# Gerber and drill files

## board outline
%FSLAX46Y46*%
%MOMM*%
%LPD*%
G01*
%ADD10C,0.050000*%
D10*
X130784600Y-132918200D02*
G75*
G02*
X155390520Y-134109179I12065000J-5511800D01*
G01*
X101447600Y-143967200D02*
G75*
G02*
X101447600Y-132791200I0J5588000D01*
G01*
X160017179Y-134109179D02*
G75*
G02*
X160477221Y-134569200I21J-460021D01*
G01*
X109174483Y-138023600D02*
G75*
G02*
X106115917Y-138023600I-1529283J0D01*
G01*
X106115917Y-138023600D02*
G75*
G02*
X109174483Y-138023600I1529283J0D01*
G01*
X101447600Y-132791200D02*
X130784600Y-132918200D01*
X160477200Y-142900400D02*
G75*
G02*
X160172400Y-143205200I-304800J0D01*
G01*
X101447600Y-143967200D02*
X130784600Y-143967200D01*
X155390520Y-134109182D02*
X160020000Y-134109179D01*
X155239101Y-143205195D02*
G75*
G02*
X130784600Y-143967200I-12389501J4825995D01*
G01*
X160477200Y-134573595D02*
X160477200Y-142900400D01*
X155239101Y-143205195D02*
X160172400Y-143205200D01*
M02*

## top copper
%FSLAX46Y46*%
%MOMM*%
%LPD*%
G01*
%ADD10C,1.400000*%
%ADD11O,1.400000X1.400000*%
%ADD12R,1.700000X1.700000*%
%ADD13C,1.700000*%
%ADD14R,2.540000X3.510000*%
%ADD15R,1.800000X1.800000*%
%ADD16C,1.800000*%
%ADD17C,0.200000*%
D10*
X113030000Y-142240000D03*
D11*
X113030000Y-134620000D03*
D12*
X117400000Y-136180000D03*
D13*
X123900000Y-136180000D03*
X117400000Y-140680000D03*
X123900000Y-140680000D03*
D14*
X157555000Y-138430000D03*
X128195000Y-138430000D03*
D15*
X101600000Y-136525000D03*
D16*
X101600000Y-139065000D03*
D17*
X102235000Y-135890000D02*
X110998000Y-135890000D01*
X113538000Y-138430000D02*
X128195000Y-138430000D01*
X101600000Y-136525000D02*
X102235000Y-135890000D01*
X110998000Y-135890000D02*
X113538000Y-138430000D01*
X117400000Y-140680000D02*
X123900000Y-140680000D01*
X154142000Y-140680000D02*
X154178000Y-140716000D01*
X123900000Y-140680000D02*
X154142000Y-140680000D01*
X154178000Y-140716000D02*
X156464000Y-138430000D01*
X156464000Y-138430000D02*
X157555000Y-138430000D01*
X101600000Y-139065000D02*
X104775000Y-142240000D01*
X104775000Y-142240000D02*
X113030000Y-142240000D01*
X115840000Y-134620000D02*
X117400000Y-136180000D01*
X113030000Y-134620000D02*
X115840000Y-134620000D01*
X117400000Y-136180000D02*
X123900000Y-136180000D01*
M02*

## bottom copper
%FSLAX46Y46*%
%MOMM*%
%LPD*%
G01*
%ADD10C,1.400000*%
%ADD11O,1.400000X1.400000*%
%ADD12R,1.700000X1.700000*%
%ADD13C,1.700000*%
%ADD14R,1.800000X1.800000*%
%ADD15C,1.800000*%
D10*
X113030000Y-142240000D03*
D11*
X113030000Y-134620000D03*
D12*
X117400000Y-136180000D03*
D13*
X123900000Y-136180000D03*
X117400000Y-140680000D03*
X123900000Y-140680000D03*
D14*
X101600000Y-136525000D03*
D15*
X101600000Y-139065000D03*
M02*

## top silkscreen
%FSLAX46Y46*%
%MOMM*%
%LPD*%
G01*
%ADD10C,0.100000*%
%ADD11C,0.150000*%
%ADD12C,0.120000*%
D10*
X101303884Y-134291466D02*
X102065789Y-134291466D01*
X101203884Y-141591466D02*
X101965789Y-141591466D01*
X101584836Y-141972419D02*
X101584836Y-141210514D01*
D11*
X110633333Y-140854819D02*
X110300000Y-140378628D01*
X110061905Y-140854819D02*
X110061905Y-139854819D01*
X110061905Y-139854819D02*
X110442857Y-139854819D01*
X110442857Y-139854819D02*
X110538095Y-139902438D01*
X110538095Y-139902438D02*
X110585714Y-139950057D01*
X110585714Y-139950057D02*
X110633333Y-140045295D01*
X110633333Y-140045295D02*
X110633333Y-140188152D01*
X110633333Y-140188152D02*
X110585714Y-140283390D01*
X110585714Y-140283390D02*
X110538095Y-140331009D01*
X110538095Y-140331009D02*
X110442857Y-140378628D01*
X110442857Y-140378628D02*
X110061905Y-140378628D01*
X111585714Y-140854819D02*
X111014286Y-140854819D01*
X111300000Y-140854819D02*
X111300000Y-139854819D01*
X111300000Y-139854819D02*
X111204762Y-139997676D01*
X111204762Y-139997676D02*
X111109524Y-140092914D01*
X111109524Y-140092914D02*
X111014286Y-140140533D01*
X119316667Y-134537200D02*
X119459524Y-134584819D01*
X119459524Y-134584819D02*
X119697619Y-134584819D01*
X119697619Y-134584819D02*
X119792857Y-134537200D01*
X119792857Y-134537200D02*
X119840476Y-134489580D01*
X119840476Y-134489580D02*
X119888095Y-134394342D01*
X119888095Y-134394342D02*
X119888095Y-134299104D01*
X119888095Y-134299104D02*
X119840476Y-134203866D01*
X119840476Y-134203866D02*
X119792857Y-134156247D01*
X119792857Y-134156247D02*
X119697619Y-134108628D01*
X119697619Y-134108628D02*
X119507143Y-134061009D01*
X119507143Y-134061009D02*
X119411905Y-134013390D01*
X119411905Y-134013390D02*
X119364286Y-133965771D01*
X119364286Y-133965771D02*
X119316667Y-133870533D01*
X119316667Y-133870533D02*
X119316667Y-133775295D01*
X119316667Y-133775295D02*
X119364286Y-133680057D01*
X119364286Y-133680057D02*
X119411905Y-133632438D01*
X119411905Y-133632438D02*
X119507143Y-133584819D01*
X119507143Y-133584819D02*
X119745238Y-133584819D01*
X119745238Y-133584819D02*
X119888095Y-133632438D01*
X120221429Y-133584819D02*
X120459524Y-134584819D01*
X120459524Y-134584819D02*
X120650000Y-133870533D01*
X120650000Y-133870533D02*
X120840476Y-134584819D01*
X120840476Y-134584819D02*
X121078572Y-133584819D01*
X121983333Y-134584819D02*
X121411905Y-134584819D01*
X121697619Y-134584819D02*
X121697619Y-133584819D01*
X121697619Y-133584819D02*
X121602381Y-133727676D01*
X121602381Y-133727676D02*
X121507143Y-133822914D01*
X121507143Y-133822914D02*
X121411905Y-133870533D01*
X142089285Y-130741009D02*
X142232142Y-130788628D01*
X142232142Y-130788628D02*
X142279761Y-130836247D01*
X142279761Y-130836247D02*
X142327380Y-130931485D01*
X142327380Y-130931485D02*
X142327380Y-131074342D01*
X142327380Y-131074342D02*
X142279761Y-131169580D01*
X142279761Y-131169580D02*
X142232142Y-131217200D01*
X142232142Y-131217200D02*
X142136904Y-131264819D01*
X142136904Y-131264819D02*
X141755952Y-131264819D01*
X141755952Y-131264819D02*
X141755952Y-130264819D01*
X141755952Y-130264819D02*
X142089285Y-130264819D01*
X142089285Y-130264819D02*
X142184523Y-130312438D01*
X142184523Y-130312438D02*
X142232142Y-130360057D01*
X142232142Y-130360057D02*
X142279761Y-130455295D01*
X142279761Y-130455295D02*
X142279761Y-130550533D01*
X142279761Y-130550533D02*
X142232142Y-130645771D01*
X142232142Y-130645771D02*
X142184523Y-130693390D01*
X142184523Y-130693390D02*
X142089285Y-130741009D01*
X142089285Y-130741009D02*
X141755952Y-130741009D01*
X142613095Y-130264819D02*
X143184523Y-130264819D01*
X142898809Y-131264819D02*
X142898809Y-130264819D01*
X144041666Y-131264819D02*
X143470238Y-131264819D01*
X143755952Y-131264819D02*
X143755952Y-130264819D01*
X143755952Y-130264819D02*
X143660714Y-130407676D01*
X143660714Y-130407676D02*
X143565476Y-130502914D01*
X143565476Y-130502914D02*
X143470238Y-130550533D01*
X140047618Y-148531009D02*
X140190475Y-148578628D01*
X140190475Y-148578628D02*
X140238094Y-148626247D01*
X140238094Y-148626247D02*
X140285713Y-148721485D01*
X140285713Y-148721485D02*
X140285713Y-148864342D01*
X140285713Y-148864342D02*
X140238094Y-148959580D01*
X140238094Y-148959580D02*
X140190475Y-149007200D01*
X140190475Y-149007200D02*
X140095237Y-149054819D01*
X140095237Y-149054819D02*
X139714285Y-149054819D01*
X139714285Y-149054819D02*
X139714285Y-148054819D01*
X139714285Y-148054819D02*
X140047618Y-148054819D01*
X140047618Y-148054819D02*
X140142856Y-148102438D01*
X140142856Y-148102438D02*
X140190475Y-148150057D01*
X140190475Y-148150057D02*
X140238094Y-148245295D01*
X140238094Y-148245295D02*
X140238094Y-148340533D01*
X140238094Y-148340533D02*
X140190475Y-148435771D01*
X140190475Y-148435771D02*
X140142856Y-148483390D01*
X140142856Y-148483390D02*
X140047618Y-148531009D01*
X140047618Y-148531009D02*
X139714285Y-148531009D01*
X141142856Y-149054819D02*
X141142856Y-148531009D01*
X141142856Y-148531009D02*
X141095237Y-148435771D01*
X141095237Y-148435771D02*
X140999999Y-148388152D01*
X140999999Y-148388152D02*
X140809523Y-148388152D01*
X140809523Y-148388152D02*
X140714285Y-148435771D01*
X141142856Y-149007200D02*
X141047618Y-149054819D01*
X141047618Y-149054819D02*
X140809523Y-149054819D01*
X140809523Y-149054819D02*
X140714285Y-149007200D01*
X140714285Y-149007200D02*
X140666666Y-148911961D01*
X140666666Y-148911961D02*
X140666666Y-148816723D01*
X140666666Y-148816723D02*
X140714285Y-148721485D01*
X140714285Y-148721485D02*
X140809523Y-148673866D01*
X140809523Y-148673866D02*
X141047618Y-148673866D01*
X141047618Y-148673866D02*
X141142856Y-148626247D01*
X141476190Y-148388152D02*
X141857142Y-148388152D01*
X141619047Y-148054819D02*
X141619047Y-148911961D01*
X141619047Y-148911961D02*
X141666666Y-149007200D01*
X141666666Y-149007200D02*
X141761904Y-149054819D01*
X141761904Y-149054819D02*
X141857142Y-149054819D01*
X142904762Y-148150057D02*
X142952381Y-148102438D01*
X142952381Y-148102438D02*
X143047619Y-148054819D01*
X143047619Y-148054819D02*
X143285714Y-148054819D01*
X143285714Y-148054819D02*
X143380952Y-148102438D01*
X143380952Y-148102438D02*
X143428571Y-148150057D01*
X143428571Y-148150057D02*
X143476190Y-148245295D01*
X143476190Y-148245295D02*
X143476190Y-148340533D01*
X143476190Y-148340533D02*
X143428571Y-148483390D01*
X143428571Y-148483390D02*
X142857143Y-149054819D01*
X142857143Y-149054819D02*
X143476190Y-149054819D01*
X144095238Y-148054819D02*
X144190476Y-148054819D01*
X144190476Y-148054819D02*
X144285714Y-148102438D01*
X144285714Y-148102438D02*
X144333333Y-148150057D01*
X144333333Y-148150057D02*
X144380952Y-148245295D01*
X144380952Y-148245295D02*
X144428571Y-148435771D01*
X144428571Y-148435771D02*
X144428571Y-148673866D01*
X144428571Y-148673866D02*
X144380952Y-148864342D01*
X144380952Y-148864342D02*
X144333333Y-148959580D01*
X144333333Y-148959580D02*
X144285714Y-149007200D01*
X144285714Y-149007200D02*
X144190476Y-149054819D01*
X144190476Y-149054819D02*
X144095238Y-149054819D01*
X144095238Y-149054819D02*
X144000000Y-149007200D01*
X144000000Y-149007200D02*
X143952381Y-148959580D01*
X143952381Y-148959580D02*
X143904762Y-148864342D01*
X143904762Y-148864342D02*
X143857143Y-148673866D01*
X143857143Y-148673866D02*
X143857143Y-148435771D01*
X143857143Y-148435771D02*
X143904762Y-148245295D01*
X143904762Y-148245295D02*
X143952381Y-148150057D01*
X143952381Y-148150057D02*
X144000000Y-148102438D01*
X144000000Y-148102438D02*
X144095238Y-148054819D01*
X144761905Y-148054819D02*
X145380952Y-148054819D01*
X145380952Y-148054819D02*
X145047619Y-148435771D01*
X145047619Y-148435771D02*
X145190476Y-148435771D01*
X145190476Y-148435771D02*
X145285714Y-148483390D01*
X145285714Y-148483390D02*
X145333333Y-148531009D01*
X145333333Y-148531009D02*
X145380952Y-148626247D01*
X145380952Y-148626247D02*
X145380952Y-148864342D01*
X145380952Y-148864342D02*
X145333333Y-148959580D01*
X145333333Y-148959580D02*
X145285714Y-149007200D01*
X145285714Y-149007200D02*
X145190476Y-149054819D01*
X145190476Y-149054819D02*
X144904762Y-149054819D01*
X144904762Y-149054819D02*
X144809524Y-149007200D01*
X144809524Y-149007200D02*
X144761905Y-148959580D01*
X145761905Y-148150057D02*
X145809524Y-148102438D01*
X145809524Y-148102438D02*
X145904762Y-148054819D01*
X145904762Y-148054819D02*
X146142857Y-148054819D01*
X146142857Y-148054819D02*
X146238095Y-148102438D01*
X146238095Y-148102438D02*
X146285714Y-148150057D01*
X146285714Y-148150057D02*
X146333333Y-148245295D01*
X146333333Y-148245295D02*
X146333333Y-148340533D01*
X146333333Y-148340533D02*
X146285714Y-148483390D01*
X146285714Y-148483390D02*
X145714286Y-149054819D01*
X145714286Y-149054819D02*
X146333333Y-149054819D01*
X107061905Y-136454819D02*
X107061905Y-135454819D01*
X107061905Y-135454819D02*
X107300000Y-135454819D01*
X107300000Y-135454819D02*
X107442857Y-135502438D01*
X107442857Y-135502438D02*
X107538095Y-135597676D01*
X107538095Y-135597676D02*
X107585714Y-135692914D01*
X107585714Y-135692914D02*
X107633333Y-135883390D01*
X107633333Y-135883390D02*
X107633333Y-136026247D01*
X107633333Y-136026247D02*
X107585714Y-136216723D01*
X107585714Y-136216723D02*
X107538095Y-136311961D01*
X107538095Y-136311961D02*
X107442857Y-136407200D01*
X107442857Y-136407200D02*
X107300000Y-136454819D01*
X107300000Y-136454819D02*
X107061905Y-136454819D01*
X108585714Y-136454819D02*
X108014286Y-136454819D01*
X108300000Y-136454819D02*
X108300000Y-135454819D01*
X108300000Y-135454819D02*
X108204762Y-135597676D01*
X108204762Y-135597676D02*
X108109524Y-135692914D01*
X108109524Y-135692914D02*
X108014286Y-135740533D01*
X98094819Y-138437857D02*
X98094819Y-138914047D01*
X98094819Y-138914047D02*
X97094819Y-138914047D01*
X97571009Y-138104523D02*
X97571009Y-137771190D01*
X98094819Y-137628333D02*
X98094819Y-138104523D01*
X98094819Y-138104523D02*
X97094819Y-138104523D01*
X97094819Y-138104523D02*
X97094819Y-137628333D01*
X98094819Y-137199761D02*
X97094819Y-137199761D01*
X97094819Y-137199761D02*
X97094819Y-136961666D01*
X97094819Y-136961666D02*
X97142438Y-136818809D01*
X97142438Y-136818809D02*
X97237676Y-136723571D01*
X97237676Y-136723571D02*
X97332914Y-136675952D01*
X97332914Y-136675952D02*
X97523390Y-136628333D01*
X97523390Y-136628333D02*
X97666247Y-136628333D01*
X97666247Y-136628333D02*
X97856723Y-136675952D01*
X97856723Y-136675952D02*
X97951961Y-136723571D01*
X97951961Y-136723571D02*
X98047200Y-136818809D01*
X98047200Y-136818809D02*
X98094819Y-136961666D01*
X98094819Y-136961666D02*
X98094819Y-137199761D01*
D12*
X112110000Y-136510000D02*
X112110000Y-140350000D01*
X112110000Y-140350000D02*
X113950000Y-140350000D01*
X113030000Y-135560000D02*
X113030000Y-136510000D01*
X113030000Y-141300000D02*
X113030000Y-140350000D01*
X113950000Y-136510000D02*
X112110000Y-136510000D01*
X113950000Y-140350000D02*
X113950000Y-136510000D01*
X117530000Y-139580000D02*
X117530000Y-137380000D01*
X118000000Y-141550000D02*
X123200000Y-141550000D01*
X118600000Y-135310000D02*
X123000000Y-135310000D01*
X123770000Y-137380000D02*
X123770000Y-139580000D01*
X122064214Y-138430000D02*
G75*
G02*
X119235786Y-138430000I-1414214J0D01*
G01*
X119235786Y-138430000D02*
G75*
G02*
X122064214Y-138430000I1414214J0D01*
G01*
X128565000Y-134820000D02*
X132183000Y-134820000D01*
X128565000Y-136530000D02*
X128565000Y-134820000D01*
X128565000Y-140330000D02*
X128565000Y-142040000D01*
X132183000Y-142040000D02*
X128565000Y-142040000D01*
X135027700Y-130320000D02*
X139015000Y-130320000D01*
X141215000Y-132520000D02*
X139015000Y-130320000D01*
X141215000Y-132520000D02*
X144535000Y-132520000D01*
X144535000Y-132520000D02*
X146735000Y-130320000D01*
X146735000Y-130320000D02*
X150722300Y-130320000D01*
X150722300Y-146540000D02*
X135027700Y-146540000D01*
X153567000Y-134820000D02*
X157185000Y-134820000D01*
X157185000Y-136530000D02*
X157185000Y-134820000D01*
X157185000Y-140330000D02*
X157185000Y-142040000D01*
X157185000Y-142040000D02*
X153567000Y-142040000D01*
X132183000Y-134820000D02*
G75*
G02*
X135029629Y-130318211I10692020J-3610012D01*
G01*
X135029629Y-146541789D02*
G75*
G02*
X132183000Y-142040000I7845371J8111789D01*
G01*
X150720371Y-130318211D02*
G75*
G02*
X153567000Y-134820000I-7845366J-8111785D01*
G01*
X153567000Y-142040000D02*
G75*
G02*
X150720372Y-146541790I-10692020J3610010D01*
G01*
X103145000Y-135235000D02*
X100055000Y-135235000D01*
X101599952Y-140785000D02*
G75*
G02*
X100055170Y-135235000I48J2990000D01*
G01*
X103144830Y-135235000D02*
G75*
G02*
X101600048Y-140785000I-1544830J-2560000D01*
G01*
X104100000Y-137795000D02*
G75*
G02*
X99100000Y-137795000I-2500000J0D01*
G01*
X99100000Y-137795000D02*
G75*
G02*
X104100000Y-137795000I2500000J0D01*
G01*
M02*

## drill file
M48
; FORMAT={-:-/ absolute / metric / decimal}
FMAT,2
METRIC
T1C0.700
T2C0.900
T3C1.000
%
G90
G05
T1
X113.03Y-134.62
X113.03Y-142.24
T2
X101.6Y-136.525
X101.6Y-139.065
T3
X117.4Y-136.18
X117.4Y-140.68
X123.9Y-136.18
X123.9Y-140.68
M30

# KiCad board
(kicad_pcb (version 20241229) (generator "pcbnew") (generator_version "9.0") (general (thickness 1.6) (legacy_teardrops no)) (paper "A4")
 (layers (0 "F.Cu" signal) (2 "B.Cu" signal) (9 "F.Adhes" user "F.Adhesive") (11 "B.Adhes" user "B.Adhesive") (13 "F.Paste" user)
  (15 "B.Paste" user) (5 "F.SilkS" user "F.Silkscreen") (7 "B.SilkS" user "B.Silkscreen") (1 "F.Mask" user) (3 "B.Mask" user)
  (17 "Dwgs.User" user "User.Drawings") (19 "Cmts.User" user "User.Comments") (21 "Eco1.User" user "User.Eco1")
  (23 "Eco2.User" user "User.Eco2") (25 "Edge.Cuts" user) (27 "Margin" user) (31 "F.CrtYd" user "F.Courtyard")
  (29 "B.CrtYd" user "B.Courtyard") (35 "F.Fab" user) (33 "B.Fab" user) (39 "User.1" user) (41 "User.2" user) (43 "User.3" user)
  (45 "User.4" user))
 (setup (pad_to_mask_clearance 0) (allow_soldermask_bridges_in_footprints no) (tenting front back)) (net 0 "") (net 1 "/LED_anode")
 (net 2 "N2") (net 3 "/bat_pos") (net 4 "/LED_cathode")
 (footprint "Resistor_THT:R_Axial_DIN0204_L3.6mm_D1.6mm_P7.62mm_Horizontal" (layer "F.Cu") (at 113.03 142.24 90)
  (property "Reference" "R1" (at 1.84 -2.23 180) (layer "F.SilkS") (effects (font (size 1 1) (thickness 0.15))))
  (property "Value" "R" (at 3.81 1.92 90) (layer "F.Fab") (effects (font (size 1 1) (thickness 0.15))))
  (fp_line (start 5.73 -0.92) (end 1.89 -0.92) (stroke (width 0.12) (type solid)) (layer "F.SilkS"))
  (fp_line (start 1.89 -0.92) (end 1.89 0.92) (stroke (width 0.12) (type solid)) (layer "F.SilkS"))
  (fp_line (start 6.68 0) (end 5.73 0) (stroke (width 0.12) (type solid)) (layer "F.SilkS"))
  (fp_line (start 0.94 0) (end 1.89 0) (stroke (width 0.12) (type solid)) (layer "F.SilkS"))
  (fp_line (start 5.73 0.92) (end 5.73 -0.92) (stroke (width 0.12) (type solid)) (layer "F.SilkS"))
  (fp_line (start 1.89 0.92) (end 5.73 0.92) (stroke (width 0.12) (type solid)) (layer "F.SilkS"))
  (pad "1" thru_hole circle (at 0 0 90) (size 1.4 1.4) (drill 0.7) (layers "*.Cu" "*.Mask") (remove_unused_layers no) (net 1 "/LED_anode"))
  (pad "2" thru_hole oval (at 7.62 0 90) (size 1.4 1.4) (drill 0.7) (layers "*.Cu" "*.Mask") (remove_unused_layers no) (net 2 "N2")))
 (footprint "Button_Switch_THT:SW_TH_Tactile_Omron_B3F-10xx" (layer "F.Cu") (at 117.4 136.18)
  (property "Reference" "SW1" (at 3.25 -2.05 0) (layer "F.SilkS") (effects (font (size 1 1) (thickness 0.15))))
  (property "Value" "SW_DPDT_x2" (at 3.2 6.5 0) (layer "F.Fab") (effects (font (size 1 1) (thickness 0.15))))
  (fp_line (start 0.13 3.4) (end 0.13 1.2) (stroke (width 0.12) (type solid)) (layer "F.SilkS"))
  (fp_line (start 0.6 5.37) (end 5.8 5.37) (stroke (width 0.12) (type solid)) (layer "F.SilkS"))
  (fp_line (start 1.2 -0.87) (end 5.6 -0.87) (stroke (width 0.12) (type solid)) (layer "F.SilkS"))
  (fp_line (start 6.37 1.2) (end 6.37 3.4) (stroke (width 0.12) (type solid)) (layer "F.SilkS"))
  (fp_circle (center 3.25 2.25) (end 4.25 3.25) (stroke (width 0.12) (type solid)) (fill no) (layer "F.SilkS"))
  (pad "1" thru_hole rect (at 0 0) (size 1.7 1.7) (drill 1) (layers "*.Cu" "*.Mask") (remove_unused_layers no) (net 2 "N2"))
  (pad "1" thru_hole circle (at 6.5 0) (size 1.7 1.7) (drill 1) (layers "*.Cu" "*.Mask") (remove_unused_layers no) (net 2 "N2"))
  (pad "2" thru_hole circle (at 0 4.5) (size 1.7 1.7) (drill 1) (layers "*.Cu" "*.Mask") (remove_unused_layers no) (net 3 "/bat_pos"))
  (pad "2" thru_hole circle (at 6.5 4.5) (size 1.7 1.7) (drill 1) (layers "*.Cu" "*.Mask") (remove_unused_layers no) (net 3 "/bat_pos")))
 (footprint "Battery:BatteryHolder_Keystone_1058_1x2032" (layer "F.Cu") (at 142.875 138.43 180)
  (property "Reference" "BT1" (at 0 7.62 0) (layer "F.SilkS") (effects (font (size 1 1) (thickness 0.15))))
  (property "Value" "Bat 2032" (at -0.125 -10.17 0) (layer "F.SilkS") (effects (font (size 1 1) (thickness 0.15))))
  (fp_line (start 14.31 3.61) (end 10.692 3.61) (stroke (width 0.12) (type solid)) (layer "F.SilkS"))
  (fp_line (start 14.31 1.9) (end 14.31 3.61) (stroke (width 0.12) (type solid)) (layer "F.SilkS"))
  (fp_line (start 14.31 -1.9) (end 14.31 -3.61) (stroke (width 0.12) (type solid)) (layer "F.SilkS"))
  (fp_line (start 10.692 -3.61) (end 14.31 -3.61) (stroke (width 0.12) (type solid)) (layer "F.SilkS"))
  (fp_line (start 7.8473 8.11) (end 3.86 8.11) (stroke (width 0.12) (type solid)) (layer "F.SilkS"))
  (fp_line (start 1.66 5.91) (end 3.86 8.11) (stroke (width 0.12) (type solid)) (layer "F.SilkS"))
  (fp_line (start 1.66 5.91) (end -1.66 5.91) (stroke (width 0.12) (type solid)) (layer "F.SilkS"))
  (fp_line (start -1.66 5.91) (end -3.86 8.11) (stroke (width 0.12) (type solid)) (layer "F.SilkS"))
  (fp_line (start -3.86 8.11) (end -7.8473 8.11) (stroke (width 0.12) (type solid)) (layer "F.SilkS"))
  (fp_line (start -7.8473 -8.11) (end 7.8473 -8.11) (stroke (width 0.12) (type solid)) (layer "F.SilkS"))
  (fp_line (start -10.692 3.61) (end -14.31 3.61) (stroke (width 0.12) (type solid)) (layer "F.SilkS"))
  (fp_line (start -14.31 1.9) (end -14.31 3.61) (stroke (width 0.12) (type solid)) (layer "F.SilkS"))
  (fp_line (start -14.31 -1.9) (end -14.31 -3.61) (stroke (width 0.12) (type solid)) (layer "F.SilkS"))
  (fp_line (start -14.31 -3.61) (end -10.692 -3.61) (stroke (width 0.12) (type solid)) (layer "F.SilkS"))
  (fp_arc (start 10.692 3.61) (mid 9.538084 6.031244) (end 7.845371 8.111789) (stroke (width 0.12) (type solid)) (layer "F.SilkS"))
  (fp_arc (start 7.845371 -8.111789) (mid 9.538085 -6.031244) (end 10.692 -3.61) (stroke (width 0.12) (type solid)) (layer "F.SilkS"))
  (fp_arc (start -7.845371 8.111789) (mid -9.538085 6.031244) (end -10.692 3.61) (stroke (width 0.12) (type solid)) (layer "F.SilkS"))
  (fp_arc (start -10.692 -3.61) (mid -9.538084 -6.031244) (end -7.845371 -8.111789) (stroke (width 0.12) (type solid)) (layer "F.SilkS"))
  (pad "1" smd rect (at -14.68 0 180) (size 2.54 3.51) (layers "F.Cu" "F.Mask" "F.Paste") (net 3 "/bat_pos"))
  (pad "2" smd rect (at 14.68 0 180) (size 2.54 3.51) (layers "F.Cu" "F.Mask" "F.Paste") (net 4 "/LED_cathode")))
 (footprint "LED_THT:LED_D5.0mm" (layer "F.Cu") (at 101.6 136.525 -90)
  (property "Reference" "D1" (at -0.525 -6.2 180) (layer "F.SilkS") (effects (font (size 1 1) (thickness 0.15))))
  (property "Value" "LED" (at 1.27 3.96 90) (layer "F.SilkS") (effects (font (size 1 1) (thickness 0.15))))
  (fp_line (start -1.29 -1.545) (end -1.29 1.545) (stroke (width 0.12) (type solid)) (layer "F.SilkS"))
  (fp_arc (start 4.26 0.000048) (mid 2.071756 2.880501) (end -1.29 1.54483) (stroke (width 0.12) (type solid)) (layer "F.SilkS"))
  (fp_arc (start -1.29 -1.54483) (mid 2.071756 -2.880501) (end 4.26 -0.000048) (stroke (width 0.12) (type solid)) (layer "F.SilkS"))
  (fp_circle (center 1.27 0) (end 3.77 0) (stroke (width 0.12) (type solid)) (fill no) (layer "F.SilkS"))
  (pad "1" thru_hole rect (at 0 0 270) (size 1.8 1.8) (drill 0.9) (layers "*.Cu" "*.Mask") (remove_unused_layers no) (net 4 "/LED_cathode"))
  (pad "2" thru_hole circle (at 2.54 0 270) (size 1.8 1.8) (drill 0.9) (layers "*.Cu" "*.Mask") (remove_unused_layers no)
   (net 1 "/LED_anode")))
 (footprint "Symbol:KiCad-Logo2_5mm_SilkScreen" (layer "B.Cu") (at 143.51 136.525 180)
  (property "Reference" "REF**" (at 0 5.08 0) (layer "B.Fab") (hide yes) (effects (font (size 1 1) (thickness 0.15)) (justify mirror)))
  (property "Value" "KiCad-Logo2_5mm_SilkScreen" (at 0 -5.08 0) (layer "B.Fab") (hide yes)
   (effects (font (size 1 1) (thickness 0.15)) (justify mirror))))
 (gr_arc (start 130.7846 132.9182) (mid 143.490874 125.181116) (end 155.39052 134.109179) (stroke (width 0.05) (type default)) (locked yes)
  (layer "Edge.Cuts"))
 (gr_arc (start 101.4476 143.9672) (mid 95.8596 138.3792) (end 101.4476 132.7912) (stroke (width 0.05) (type default)) (locked yes)
  (layer "Edge.Cuts"))
 (gr_arc (start 160.017179 134.109179) (mid 160.342463 134.243916) (end 160.4772 134.5692) (stroke (width 0.05) (type default)) (locked yes)
  (layer "Edge.Cuts"))
 (gr_circle (center 107.6452 138.0236) (end 108.7882 139.0396) (stroke (width 0.05) (type default)) (fill no) (layer "Edge.Cuts"))
 (gr_line (start 101.4476 132.7912) (end 130.7846 132.9182) (stroke (width 0.05) (type default)) (locked yes) (layer "Edge.Cuts"))
 (gr_arc (start 160.4772 142.9004) (mid 160.387926 143.115926) (end 160.1724 143.2052) (stroke (width 0.05) (type default)) (locked yes)
  (layer "Edge.Cuts"))
 (gr_line (start 101.4476 143.9672) (end 130.7846 143.9672) (stroke (width 0.05) (type default)) (locked yes) (layer "Edge.Cuts"))
 (gr_line (start 155.39052 134.109182) (end 160.02 134.109179) (stroke (width 0.05) (type default)) (locked yes) (layer "Edge.Cuts"))
 (gr_arc (start 155.239101 143.205195) (mid 143.263711 151.668988) (end 130.7846 143.9672) (stroke (width 0.05) (type default)) (locked yes)
  (layer "Edge.Cuts"))
 (gr_line (start 160.4772 134.573595) (end 160.4772 142.9004) (stroke (width 0.05) (type default)) (locked yes) (layer "Edge.Cuts"))
 (gr_line (start 155.239101 143.205195) (end 160.1724 143.2052) (stroke (width 0.05) (type default)) (locked yes) (layer "Edge.Cuts"))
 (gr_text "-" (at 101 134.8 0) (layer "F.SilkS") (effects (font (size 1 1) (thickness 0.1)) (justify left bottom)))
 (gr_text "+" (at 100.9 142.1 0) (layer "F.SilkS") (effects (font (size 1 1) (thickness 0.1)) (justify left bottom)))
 (segment (start 102.235 135.89) (end 110.998 135.89) (width 0.2) (layer "F.Cu") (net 4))
 (segment (start 113.538 138.43) (end 128.195 138.43) (width 0.2) (layer "F.Cu") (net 4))
 (segment (start 101.6 136.525) (end 102.235 135.89) (width 0.2) (layer "F.Cu") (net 4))
 (segment (start 110.998 135.89) (end 113.538 138.43) (width 0.2) (layer "F.Cu") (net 4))
 (segment (start 117.4 140.68) (end 123.9 140.68) (width 0.2) (layer "F.Cu") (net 3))
 (segment (start 154.142 140.68) (end 154.178 140.716) (width 0.2) (layer "F.Cu") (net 3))
 (segment (start 123.9 140.68) (end 154.142 140.68) (width 0.2) (layer "F.Cu") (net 3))
 (segment (start 154.178 140.716) (end 156.464 138.43) (width 0.2) (layer "F.Cu") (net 3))
 (segment (start 156.464 138.43) (end 157.555 138.43) (width 0.2) (layer "F.Cu") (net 3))
 (segment (start 101.6 139.065) (end 104.775 142.24) (width 0.2) (layer "F.Cu") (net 1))
 (segment (start 104.775 142.24) (end 113.03 142.24) (width 0.2) (layer "F.Cu") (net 1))
 (segment (start 115.84 134.62) (end 117.4 136.18) (width 0.2) (layer "F.Cu") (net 2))
 (segment (start 113.03 134.62) (end 115.84 134.62) (width 0.2) (layer "F.Cu") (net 2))
 (segment (start 117.4 136.18) (end 123.9 136.18) (width 0.2) (layer "F.Cu") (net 2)))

